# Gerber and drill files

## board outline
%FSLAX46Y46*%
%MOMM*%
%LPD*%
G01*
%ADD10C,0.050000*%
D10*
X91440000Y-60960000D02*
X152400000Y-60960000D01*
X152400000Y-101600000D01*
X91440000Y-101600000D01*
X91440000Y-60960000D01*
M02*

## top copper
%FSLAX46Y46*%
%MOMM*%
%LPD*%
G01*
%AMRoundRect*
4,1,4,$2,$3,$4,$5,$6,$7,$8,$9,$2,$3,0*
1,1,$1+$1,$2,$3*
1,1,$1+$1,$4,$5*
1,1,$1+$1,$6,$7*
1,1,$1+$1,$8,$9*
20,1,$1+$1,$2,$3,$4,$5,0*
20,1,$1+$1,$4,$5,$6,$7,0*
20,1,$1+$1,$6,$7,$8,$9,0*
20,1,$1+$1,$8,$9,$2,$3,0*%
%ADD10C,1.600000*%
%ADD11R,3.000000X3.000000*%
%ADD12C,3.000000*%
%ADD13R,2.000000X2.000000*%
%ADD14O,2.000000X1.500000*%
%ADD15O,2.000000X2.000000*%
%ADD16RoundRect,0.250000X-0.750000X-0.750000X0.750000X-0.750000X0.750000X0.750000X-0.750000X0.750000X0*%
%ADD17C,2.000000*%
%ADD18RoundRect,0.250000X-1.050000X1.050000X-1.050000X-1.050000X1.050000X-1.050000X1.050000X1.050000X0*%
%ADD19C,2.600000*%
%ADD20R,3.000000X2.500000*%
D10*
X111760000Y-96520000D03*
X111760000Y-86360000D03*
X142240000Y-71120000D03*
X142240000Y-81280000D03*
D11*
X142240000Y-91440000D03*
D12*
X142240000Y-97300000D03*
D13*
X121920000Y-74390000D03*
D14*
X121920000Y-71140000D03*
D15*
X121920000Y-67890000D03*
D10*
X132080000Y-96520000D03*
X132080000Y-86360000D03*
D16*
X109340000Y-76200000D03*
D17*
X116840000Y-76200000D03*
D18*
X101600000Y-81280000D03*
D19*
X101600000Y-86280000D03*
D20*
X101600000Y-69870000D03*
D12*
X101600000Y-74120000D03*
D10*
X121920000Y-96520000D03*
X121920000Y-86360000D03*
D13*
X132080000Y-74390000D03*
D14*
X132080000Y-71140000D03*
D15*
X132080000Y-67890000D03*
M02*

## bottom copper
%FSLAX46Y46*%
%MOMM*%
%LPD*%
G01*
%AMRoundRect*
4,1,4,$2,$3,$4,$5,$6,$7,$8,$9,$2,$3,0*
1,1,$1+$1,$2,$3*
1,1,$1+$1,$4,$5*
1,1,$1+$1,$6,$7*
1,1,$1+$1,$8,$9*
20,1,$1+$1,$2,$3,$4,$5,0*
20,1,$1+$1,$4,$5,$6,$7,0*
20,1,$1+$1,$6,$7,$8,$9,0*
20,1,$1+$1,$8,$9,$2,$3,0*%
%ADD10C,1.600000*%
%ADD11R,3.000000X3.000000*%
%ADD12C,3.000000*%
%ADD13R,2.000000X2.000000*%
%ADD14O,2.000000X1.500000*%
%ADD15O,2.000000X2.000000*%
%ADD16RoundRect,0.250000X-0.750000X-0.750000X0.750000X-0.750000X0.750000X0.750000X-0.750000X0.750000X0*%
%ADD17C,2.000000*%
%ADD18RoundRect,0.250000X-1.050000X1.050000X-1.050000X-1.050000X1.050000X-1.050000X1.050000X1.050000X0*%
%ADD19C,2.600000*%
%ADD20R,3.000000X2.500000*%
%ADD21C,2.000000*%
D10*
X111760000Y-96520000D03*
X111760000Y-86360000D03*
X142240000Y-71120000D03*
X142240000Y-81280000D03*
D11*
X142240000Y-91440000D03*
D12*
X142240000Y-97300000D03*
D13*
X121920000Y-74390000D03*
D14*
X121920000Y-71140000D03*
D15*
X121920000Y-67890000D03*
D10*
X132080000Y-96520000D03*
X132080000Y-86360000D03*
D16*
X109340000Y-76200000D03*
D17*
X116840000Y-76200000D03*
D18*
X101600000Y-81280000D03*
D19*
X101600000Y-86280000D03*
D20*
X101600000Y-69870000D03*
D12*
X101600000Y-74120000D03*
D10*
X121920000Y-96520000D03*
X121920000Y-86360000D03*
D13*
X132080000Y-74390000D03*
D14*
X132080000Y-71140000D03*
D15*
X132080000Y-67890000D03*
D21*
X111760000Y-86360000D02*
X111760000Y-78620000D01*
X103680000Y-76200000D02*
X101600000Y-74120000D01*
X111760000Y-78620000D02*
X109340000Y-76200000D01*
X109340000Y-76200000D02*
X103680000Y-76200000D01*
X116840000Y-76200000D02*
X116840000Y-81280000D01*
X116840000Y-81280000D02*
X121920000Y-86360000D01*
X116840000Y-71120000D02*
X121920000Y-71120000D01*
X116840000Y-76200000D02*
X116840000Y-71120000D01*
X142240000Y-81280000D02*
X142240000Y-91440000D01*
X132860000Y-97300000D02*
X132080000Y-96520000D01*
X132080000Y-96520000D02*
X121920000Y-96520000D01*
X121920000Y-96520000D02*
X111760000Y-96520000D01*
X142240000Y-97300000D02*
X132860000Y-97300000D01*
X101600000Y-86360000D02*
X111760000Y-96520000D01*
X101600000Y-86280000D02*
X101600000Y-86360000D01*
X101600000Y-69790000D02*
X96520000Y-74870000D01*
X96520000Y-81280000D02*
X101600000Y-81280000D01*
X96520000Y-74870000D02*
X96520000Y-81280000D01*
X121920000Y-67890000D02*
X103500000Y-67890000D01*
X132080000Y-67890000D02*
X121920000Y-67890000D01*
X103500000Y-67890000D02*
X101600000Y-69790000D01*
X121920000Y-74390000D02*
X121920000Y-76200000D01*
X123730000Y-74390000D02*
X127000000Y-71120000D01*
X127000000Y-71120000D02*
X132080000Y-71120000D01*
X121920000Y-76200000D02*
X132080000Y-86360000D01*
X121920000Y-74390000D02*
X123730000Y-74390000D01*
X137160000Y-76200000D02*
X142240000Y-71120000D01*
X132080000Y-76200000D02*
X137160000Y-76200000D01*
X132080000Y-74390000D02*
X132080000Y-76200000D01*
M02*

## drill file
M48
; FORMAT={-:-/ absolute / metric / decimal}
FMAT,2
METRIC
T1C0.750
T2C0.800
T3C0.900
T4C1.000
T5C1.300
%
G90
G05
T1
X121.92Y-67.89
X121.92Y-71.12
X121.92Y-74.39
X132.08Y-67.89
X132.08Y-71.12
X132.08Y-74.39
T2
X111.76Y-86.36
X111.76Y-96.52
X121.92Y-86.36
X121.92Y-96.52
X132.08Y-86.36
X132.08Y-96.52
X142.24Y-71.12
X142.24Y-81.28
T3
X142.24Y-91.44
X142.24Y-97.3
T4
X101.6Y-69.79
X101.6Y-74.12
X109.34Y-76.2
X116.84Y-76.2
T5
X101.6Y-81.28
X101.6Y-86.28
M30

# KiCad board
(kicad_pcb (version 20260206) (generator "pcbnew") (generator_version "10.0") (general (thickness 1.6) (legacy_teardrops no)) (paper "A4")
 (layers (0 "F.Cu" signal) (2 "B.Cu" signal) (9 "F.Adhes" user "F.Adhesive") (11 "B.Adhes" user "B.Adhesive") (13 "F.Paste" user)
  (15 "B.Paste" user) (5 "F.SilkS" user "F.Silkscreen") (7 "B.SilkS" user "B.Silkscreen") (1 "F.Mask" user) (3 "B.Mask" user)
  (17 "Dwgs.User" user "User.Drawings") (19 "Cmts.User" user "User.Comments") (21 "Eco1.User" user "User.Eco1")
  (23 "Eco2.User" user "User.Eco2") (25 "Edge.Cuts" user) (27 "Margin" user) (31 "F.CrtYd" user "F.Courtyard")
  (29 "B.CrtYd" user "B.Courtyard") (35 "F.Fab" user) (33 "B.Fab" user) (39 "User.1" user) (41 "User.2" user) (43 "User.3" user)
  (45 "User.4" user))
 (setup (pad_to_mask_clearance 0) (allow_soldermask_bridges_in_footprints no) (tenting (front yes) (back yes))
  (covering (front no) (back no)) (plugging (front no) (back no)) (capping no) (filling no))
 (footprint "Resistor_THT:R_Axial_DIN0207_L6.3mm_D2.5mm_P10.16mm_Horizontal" (layer "F.Cu") (at 111.76 96.52 90)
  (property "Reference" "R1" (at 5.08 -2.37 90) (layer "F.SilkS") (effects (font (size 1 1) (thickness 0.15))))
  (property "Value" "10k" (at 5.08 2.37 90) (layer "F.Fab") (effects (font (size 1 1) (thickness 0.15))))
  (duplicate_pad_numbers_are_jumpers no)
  (pad "1" thru_hole circle (at 0 0 90) (size 1.6 1.6) (drill 0.8) (layers "*.Cu" "*.Mask") (remove_unused_layers no) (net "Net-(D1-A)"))
  (pad "2" thru_hole circle (at 10.16 0 90) (size 1.6 1.6) (drill 0.8) (layers "*.Cu" "*.Mask") (remove_unused_layers no)
   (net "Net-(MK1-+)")))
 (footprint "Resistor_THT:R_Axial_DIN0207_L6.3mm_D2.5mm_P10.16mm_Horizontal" (layer "F.Cu") (at 142.24 71.12 -90)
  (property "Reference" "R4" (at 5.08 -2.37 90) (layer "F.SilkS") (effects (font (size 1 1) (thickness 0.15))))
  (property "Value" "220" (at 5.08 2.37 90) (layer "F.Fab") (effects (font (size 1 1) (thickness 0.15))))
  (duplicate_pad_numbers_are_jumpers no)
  (pad "1" thru_hole circle (at 0 0 270) (size 1.6 1.6) (drill 0.8) (layers "*.Cu" "*.Mask") (remove_unused_layers no) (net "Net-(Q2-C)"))
  (pad "2" thru_hole circle (at 10.16 0 270) (size 1.6 1.6) (drill 0.8) (layers "*.Cu" "*.Mask") (remove_unused_layers no)
   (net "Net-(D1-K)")))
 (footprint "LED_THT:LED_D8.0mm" (layer "F.Cu") (at 142.24 91.44 -90)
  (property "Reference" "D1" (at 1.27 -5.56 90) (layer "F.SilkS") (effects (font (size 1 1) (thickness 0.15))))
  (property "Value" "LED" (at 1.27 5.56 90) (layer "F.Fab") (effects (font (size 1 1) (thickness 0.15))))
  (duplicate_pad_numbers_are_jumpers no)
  (pad "1" thru_hole rect (at 0 0 270) (size 3 3) (drill 0.9) (layers "*.Cu" "*.Mask") (remove_unused_layers no) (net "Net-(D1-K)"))
  (pad "2" thru_hole circle (at 5.86 0 270) (size 3 3) (drill 0.9) (layers "*.Cu" "*.Mask") (remove_unused_layers no) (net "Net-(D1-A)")))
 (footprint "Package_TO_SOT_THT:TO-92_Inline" (layer "F.Cu") (at 121.92 72.39 90)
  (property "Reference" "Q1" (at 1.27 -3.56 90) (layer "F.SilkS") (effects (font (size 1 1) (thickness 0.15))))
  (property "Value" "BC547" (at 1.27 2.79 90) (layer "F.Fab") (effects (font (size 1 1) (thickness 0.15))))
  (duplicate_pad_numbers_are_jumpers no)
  (pad "1" thru_hole rect (at -2 0 90) (size 2 2) (drill 0.75) (layers "*.Cu" "*.Mask") (remove_unused_layers no) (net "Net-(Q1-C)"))
  (pad "2" thru_hole oval (at 1.27 0 90) (size 1.5 2) (drill 0.75 (offset -0.02 0)) (layers "*.Cu" "*.Mask") (remove_unused_layers no)
   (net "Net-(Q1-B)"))
  (pad "3" thru_hole oval (at 4.5 0 90) (size 2 2) (drill 0.75) (layers "*.Cu" "*.Mask") (remove_unused_layers no) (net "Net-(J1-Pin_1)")))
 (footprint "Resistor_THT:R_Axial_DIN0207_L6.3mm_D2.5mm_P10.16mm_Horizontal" (layer "F.Cu") (at 132.08 96.52 90)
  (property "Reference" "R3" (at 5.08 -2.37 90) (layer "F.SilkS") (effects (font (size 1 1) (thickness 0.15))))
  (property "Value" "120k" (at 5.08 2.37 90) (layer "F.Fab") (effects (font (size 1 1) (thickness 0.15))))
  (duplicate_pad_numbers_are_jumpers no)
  (pad "1" thru_hole circle (at 0 0 90) (size 1.6 1.6) (drill 0.8) (layers "*.Cu" "*.Mask") (remove_unused_layers no) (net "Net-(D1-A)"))
  (pad "2" thru_hole circle (at 10.16 0 90) (size 1.6 1.6) (drill 0.8) (layers "*.Cu" "*.Mask") (remove_unused_layers no) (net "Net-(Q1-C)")))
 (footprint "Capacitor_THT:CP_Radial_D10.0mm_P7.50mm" (layer "F.Cu") (at 109.34 76.2)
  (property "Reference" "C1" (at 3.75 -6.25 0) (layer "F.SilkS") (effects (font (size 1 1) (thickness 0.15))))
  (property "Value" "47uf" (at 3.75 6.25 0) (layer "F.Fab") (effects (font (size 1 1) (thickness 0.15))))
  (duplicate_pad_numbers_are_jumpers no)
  (pad "1" thru_hole roundrect (at 0 0) (size 2 2) (drill 1) (layers "*.Cu" "*.Mask") (remove_unused_layers no) (roundrect_rratio 0.125)
   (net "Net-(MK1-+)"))
  (pad "2" thru_hole circle (at 7.5 0) (size 2 2) (drill 1) (layers "*.Cu" "*.Mask") (remove_unused_layers no) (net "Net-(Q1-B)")))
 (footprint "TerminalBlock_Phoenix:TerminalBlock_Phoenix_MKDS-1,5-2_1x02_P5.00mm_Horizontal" (layer "F.Cu") (at 101.6 81.28 -90)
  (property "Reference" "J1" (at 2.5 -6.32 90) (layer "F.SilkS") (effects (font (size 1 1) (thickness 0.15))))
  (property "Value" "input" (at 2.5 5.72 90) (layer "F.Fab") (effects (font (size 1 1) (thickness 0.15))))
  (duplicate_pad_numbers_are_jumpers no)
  (pad "1" thru_hole roundrect (at 0 0 270) (size 2.6 2.6) (drill 1.3) (layers "*.Cu" "*.Mask") (remove_unused_layers no)
   (roundrect_rratio 0.096154) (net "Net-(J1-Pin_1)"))
  (pad "2" thru_hole circle (at 5 0 270) (size 2.6 2.6) (drill 1.3) (layers "*.Cu" "*.Mask") (remove_unused_layers no) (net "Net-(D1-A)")))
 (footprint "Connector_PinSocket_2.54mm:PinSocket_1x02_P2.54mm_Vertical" (layer "F.Cu") (at 101.6 71.12)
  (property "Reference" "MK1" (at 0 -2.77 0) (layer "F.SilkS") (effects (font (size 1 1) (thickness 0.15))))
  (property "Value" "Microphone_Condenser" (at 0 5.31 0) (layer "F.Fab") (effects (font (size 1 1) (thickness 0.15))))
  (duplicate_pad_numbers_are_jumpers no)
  (pad "1" thru_hole rect (at 0 -1.33) (size 3 2.5) (drill 1 (offset 0 0.08)) (layers "*.Cu" "*.Mask") (remove_unused_layers no)
   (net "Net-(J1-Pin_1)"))
  (pad "2" thru_hole circle (at 0 3) (size 3 3) (drill 1) (layers "*.Cu" "*.Mask") (remove_unused_layers no) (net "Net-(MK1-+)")))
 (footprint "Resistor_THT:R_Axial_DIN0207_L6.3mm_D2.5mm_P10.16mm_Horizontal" (layer "F.Cu") (at 121.92 96.52 90)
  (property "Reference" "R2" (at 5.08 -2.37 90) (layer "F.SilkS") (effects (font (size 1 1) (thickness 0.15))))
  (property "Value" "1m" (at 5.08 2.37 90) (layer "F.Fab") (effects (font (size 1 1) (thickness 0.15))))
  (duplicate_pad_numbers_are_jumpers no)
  (pad "1" thru_hole circle (at 0 0 90) (size 1.6 1.6) (drill 0.8) (layers "*.Cu" "*.Mask") (remove_unused_layers no) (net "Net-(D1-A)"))
  (pad "2" thru_hole circle (at 10.16 0 90) (size 1.6 1.6) (drill 0.8) (layers "*.Cu" "*.Mask") (remove_unused_layers no) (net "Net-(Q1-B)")))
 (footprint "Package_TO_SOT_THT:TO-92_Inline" (layer "F.Cu") (at 132.08 72.39 90)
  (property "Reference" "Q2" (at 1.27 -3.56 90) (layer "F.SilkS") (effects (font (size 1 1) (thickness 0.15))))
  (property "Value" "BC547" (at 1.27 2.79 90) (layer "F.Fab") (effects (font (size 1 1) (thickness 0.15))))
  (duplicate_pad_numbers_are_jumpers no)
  (pad "1" thru_hole rect (at -2 0 90) (size 2 2) (drill 0.75) (layers "*.Cu" "*.Mask") (remove_unused_layers no) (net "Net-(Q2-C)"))
  (pad "2" thru_hole oval (at 1.27 0 90) (size 1.5 2) (drill 0.75 (offset -0.02 0)) (layers "*.Cu" "*.Mask") (remove_unused_layers no)
   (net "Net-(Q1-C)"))
  (pad "3" thru_hole oval (at 4.5 0 90) (size 2 2) (drill 0.75) (layers "*.Cu" "*.Mask") (remove_unused_layers no) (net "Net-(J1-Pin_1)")))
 (gr_rect (start 91.44 60.96) (end 152.4 101.6) (stroke (width 0.05) (type default)) (fill no) (layer "Edge.Cuts"))
 (segment (start 111.76 86.36) (end 111.76 78.62) (width 2) (layer "B.Cu") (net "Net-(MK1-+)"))
 (segment (start 103.68 76.2) (end 101.6 74.12) (width 2) (layer "B.Cu") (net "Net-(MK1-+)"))
 (segment (start 111.76 78.62) (end 109.34 76.2) (width 2) (layer "B.Cu") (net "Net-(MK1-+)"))
 (segment (start 109.34 76.2) (end 103.68 76.2) (width 2) (layer "B.Cu") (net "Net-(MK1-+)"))
 (segment (start 116.84 76.2) (end 116.84 81.28) (width 2) (layer "B.Cu") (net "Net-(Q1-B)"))
 (segment (start 116.84 81.28) (end 121.92 86.36) (width 2) (layer "B.Cu") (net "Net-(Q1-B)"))
 (segment (start 116.84 71.12) (end 121.92 71.12) (width 2) (layer "B.Cu") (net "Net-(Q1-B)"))
 (segment (start 116.84 76.2) (end 116.84 71.12) (width 2) (layer "B.Cu") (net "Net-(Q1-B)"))
 (segment (start 142.24 81.28) (end 142.24 91.44) (width 2) (layer "B.Cu") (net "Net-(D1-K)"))
 (segment (start 132.86 97.3) (end 132.08 96.52) (width 2) (layer "B.Cu") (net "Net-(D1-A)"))
 (segment (start 132.08 96.52) (end 121.92 96.52) (width 2) (layer "B.Cu") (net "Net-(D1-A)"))
 (segment (start 121.92 96.52) (end 111.76 96.52) (width 2) (layer "B.Cu") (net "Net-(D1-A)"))
 (segment (start 142.24 97.3) (end 132.86 97.3) (width 2) (layer "B.Cu") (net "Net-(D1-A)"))
 (segment (start 101.6 86.36) (end 111.76 96.52) (width 2) (layer "B.Cu") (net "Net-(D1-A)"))
 (segment (start 101.6 86.28) (end 101.6 86.36) (width 2) (layer "B.Cu") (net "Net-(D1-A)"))
 (segment (start 101.6 69.79) (end 96.52 74.87) (width 2) (layer "B.Cu") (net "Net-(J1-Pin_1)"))
 (segment (start 96.52 81.28) (end 101.6 81.28) (width 2) (layer "B.Cu") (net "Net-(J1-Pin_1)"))
 (segment (start 96.52 74.87) (end 96.52 81.28) (width 2) (layer "B.Cu") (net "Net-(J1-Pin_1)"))
 (segment (start 121.92 67.89) (end 103.5 67.89) (width 2) (layer "B.Cu") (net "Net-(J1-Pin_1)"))
 (segment (start 132.08 67.89) (end 121.92 67.89) (width 2) (layer "B.Cu") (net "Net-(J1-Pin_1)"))
 (segment (start 103.5 67.89) (end 101.6 69.79) (width 2) (layer "B.Cu") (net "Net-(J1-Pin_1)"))
 (segment (start 121.92 74.39) (end 121.92 76.2) (width 2) (layer "B.Cu") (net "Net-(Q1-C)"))
 (segment (start 123.73 74.39) (end 127 71.12) (width 2) (layer "B.Cu") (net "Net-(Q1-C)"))
 (segment (start 127 71.12) (end 132.08 71.12) (width 2) (layer "B.Cu") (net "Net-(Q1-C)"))
 (segment (start 121.92 76.2) (end 132.08 86.36) (width 2) (layer "B.Cu") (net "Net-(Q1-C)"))
 (segment (start 121.92 74.39) (end 123.73 74.39) (width 2) (layer "B.Cu") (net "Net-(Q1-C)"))
 (segment (start 137.16 76.2) (end 142.24 71.12) (width 2) (layer "B.Cu") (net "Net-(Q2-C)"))
 (segment (start 132.08 76.2) (end 137.16 76.2) (width 2) (layer "B.Cu") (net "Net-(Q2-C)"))
 (segment (start 132.08 74.39) (end 132.08 76.2) (width 2) (layer "B.Cu") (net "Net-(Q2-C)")))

